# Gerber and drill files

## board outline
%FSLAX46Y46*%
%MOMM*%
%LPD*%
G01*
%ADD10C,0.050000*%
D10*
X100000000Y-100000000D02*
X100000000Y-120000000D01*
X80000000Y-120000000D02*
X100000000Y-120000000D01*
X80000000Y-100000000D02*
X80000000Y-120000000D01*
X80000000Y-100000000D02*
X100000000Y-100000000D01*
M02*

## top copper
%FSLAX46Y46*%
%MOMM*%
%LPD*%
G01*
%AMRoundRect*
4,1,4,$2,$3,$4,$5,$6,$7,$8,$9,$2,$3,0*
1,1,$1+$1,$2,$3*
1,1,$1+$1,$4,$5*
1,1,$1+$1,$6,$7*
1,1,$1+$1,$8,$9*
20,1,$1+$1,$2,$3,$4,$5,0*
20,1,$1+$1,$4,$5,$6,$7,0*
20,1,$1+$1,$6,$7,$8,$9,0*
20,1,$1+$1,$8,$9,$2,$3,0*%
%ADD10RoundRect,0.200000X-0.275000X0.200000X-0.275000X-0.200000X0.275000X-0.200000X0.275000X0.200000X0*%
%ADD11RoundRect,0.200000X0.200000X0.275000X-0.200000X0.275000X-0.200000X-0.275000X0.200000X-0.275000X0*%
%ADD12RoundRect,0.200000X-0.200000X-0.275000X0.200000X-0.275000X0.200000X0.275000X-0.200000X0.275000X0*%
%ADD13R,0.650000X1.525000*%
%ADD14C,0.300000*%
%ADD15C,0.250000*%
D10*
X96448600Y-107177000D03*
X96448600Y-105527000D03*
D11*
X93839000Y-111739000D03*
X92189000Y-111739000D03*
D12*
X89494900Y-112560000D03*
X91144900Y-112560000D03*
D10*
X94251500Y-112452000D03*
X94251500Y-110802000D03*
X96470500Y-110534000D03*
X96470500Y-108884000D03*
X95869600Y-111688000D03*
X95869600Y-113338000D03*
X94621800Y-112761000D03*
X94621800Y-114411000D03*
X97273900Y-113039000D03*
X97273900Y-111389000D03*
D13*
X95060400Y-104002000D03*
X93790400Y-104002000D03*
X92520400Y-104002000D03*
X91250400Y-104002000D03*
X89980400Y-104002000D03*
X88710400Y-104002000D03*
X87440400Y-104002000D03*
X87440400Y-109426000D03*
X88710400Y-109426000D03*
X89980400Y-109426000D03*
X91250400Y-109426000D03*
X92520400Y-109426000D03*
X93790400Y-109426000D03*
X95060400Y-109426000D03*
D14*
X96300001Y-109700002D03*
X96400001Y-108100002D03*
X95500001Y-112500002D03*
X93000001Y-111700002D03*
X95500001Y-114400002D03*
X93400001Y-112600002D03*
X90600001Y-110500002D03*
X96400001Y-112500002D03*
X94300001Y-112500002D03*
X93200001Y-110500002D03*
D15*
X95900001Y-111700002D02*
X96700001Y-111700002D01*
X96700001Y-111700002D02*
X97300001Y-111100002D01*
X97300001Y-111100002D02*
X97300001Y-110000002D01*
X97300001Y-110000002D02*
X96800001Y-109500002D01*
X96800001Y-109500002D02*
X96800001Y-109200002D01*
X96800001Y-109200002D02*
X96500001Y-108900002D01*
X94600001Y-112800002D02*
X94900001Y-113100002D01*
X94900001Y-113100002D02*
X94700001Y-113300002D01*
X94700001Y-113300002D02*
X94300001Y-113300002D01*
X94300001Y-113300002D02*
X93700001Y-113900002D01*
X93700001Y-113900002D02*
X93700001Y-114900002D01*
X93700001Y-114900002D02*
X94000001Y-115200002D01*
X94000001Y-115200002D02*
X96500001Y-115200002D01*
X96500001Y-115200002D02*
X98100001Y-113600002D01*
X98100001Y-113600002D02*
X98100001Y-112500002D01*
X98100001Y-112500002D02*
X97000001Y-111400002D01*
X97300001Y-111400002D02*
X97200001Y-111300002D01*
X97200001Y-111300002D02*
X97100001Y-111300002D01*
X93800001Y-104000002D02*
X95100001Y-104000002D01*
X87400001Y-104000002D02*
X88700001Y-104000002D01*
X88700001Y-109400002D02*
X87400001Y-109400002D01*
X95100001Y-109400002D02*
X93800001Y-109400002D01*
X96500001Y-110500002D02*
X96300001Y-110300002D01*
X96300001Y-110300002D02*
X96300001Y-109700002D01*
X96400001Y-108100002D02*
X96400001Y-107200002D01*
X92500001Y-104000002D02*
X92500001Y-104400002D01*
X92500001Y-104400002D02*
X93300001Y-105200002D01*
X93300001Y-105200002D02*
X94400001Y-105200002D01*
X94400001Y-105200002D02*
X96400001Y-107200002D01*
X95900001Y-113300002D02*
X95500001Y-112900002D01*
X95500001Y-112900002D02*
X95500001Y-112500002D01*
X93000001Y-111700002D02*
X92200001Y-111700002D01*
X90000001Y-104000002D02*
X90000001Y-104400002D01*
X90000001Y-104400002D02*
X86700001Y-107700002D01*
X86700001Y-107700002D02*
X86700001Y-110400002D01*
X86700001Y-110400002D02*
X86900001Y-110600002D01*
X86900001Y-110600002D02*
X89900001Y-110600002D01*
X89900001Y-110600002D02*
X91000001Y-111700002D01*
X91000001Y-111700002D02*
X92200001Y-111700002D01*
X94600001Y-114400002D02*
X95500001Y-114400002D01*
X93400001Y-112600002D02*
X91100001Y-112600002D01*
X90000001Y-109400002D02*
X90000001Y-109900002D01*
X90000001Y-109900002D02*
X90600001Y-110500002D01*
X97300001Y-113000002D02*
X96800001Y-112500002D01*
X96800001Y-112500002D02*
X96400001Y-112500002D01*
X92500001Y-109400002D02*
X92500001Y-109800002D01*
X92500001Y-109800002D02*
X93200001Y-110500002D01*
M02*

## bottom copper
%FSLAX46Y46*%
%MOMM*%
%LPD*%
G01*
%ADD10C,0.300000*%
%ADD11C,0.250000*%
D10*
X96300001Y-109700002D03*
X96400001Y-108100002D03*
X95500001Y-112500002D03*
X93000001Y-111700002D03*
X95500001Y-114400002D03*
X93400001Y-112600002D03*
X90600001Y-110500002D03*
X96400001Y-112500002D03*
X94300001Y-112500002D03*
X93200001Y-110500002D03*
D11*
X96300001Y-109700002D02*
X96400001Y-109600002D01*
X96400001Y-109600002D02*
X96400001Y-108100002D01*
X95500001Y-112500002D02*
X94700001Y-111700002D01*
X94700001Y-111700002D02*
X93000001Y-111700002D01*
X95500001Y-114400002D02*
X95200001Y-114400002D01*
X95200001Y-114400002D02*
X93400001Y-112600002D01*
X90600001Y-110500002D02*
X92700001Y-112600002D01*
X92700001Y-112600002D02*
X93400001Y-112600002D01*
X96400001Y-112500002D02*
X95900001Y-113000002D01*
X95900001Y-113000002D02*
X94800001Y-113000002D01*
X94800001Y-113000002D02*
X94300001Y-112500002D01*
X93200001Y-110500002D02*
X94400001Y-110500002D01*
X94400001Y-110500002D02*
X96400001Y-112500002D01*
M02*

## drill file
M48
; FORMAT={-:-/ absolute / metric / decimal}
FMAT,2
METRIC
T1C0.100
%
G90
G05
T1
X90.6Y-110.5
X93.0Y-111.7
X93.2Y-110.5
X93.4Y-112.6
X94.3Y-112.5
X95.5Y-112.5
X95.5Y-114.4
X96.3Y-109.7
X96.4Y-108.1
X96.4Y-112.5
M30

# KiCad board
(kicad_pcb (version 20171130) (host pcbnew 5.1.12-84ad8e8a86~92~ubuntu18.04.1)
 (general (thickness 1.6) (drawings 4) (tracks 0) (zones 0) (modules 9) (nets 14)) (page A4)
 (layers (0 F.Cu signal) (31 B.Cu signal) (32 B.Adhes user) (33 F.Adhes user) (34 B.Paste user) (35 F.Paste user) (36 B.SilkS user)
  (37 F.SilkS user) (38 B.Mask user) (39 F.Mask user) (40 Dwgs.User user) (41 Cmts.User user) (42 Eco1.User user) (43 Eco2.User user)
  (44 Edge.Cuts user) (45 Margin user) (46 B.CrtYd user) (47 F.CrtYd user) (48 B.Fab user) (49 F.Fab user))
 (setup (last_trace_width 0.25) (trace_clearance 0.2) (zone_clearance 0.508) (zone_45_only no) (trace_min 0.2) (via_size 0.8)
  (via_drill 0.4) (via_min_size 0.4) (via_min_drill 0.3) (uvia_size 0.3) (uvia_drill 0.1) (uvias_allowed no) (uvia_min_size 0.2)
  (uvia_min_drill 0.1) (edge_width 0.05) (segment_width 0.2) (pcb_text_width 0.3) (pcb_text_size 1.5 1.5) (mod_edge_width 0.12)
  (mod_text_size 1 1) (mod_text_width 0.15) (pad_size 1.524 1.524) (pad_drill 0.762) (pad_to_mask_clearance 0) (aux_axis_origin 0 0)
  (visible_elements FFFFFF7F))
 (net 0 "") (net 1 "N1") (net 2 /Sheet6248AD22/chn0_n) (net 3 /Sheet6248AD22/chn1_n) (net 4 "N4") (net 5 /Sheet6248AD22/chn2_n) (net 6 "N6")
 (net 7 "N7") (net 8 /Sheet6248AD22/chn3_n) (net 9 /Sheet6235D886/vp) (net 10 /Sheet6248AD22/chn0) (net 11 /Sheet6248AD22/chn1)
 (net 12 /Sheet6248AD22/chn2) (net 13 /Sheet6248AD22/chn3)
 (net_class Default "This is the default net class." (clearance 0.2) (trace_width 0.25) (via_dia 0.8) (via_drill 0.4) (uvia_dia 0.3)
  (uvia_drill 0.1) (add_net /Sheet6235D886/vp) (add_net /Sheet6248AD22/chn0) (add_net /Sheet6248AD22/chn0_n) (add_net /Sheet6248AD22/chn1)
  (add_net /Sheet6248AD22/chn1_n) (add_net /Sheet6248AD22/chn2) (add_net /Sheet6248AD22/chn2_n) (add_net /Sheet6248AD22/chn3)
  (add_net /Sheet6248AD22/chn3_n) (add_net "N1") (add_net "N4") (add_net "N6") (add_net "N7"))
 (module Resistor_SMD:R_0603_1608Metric (layer F.Cu) (at 96.448600 106.352000 270.000000)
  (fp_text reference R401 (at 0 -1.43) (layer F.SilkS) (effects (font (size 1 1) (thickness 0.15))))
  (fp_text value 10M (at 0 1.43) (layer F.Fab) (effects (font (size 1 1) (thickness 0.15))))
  (pad 2 smd roundrect (at 0.825 0 270.000000) (size 0.8 0.95) (layers F.Cu F.Mask F.Paste) (roundrect_rratio 0.25) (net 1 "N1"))
  (pad 1 smd roundrect (at -0.825 0 270.000000) (size 0.8 0.95) (layers F.Cu F.Mask F.Paste) (roundrect_rratio 0.25)
   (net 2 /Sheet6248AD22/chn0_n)))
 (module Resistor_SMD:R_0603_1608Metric (layer F.Cu) (at 93.014000 111.739000 180.000000)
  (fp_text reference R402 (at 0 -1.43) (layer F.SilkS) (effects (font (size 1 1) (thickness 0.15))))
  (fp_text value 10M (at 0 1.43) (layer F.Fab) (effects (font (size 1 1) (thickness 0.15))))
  (pad 1 smd roundrect (at -0.825 0 180.000000) (size 0.8 0.95) (layers F.Cu F.Mask F.Paste) (roundrect_rratio 0.25)
   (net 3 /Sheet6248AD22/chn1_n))
  (pad 2 smd roundrect (at 0.825 0 180.000000) (size 0.8 0.95) (layers F.Cu F.Mask F.Paste) (roundrect_rratio 0.25) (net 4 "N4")))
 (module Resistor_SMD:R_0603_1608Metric (layer F.Cu) (at 90.319900 112.560000)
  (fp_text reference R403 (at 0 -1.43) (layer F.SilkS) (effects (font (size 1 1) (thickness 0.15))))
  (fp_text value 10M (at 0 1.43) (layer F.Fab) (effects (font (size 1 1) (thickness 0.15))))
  (pad 1 smd roundrect (at -0.825 0) (size 0.8 0.95) (layers F.Cu F.Mask F.Paste) (roundrect_rratio 0.25) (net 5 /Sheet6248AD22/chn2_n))
  (pad 2 smd roundrect (at 0.825 0) (size 0.8 0.95) (layers F.Cu F.Mask F.Paste) (roundrect_rratio 0.25) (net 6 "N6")))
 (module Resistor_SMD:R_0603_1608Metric (layer F.Cu) (at 94.251500 111.627000 270.000000)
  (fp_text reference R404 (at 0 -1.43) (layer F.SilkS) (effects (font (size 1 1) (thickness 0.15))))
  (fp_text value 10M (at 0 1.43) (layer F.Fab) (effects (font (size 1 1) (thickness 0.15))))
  (pad 2 smd roundrect (at 0.825 0 270.000000) (size 0.8 0.95) (layers F.Cu F.Mask F.Paste) (roundrect_rratio 0.25) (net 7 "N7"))
  (pad 1 smd roundrect (at -0.825 0 270.000000) (size 0.8 0.95) (layers F.Cu F.Mask F.Paste) (roundrect_rratio 0.25)
   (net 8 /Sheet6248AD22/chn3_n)))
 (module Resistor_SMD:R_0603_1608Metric (layer F.Cu) (at 96.470500 109.709000 270.000000)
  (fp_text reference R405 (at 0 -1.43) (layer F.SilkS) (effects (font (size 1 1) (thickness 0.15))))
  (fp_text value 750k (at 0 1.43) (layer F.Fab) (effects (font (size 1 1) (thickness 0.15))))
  (pad 2 smd roundrect (at 0.825 0 270.000000) (size 0.8 0.95) (layers F.Cu F.Mask F.Paste) (roundrect_rratio 0.25) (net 1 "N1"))
  (pad 1 smd roundrect (at -0.825 0 270.000000) (size 0.8 0.95) (layers F.Cu F.Mask F.Paste) (roundrect_rratio 0.25)
   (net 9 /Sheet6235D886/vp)))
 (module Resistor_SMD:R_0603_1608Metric (layer F.Cu) (at 95.869600 112.513000 270.000000)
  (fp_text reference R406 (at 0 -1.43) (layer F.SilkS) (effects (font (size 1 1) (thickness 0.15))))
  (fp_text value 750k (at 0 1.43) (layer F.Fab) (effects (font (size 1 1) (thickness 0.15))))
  (pad 1 smd roundrect (at -0.825 0 270.000000) (size 0.8 0.95) (layers F.Cu F.Mask F.Paste) (roundrect_rratio 0.25)
   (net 9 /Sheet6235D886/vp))
  (pad 2 smd roundrect (at 0.825 0 270.000000) (size 0.8 0.95) (layers F.Cu F.Mask F.Paste) (roundrect_rratio 0.25) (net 4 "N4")))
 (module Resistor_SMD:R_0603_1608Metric (layer F.Cu) (at 94.621800 113.586000 270.000000)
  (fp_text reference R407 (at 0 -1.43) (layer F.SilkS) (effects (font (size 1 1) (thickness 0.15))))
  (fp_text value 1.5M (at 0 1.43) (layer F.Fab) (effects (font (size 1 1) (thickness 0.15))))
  (pad 1 smd roundrect (at -0.825 0 270.000000) (size 0.8 0.95) (layers F.Cu F.Mask F.Paste) (roundrect_rratio 0.25)
   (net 9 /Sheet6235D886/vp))
  (pad 2 smd roundrect (at 0.825 0 270.000000) (size 0.8 0.95) (layers F.Cu F.Mask F.Paste) (roundrect_rratio 0.25) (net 6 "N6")))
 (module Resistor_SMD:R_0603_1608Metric (layer F.Cu) (at 97.273900 112.214000 270.000000)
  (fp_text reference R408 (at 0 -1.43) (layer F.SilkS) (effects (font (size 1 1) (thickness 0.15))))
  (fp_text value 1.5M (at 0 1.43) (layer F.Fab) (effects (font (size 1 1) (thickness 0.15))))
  (pad 2 smd roundrect (at 0.825 0 270.000000) (size 0.8 0.95) (layers F.Cu F.Mask F.Paste) (roundrect_rratio 0.25) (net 7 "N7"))
  (pad 1 smd roundrect (at -0.825 0 270.000000) (size 0.8 0.95) (layers F.Cu F.Mask F.Paste) (roundrect_rratio 0.25)
   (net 9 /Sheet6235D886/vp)))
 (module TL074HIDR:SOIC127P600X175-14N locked (layer F.Cu) (at 91.250400 106.714000 270.000000)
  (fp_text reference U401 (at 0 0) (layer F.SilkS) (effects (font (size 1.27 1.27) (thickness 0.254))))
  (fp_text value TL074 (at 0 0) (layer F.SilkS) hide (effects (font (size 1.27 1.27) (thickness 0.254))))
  (pad 1 smd rect (at -2.712 -3.81) (size 0.65 1.525) (layers F.Cu F.Mask F.Paste) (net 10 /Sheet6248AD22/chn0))
  (pad 2 smd rect (at -2.712 -2.54) (size 0.65 1.525) (layers F.Cu F.Mask F.Paste) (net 10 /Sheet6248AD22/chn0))
  (pad 3 smd rect (at -2.712 -1.27) (size 0.65 1.525) (layers F.Cu F.Mask F.Paste) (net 1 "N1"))
  (pad 4 smd rect (at -2.712 0) (size 0.65 1.525) (layers F.Cu F.Mask F.Paste))
  (pad 5 smd rect (at -2.712 1.27) (size 0.65 1.525) (layers F.Cu F.Mask F.Paste) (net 4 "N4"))
  (pad 6 smd rect (at -2.712 2.54) (size 0.65 1.525) (layers F.Cu F.Mask F.Paste) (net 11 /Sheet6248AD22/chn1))
  (pad 7 smd rect (at -2.712 3.81) (size 0.65 1.525) (layers F.Cu F.Mask F.Paste) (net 11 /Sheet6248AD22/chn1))
  (pad 8 smd rect (at 2.712 3.81) (size 0.65 1.525) (layers F.Cu F.Mask F.Paste) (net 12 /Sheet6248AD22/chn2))
  (pad 9 smd rect (at 2.712 2.54) (size 0.65 1.525) (layers F.Cu F.Mask F.Paste) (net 12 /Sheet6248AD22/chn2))
  (pad 10 smd rect (at 2.712 1.27) (size 0.65 1.525) (layers F.Cu F.Mask F.Paste) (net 6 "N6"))
  (pad 11 smd rect (at 2.712 0) (size 0.65 1.525) (layers F.Cu F.Mask F.Paste))
  (pad 12 smd rect (at 2.712 -1.27) (size 0.65 1.525) (layers F.Cu F.Mask F.Paste) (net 7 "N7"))
  (pad 13 smd rect (at 2.712 -2.54) (size 0.65 1.525) (layers F.Cu F.Mask F.Paste) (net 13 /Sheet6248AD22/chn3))
  (pad 14 smd rect (at 2.712 -3.81) (size 0.65 1.525) (layers F.Cu F.Mask F.Paste) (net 13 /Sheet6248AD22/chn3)))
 (gr_line (start 100 100) (end 100 120) (layer Edge.Cuts) (width 0.05))
 (gr_line (start 80 120) (end 100 120) (layer Edge.Cuts) (width 0.05))
 (gr_line (start 80 100) (end 80 120) (layer Edge.Cuts) (width 0.05))
 (gr_line (start 80 100) (end 100 100) (layer Edge.Cuts) (width 0.05))
 (segment (start 95.900001 111.700002) (end 96.700001 111.700002) (width 0.250000) (layer F.Cu) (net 9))
 (segment (start 96.700001 111.700002) (end 97.300001 111.100002) (width 0.250000) (layer F.Cu) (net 9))
 (segment (start 97.300001 111.100002) (end 97.300001 110.000002) (width 0.250000) (layer F.Cu) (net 9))
 (segment (start 97.300001 110.000002) (end 96.800001 109.500002) (width 0.250000) (layer F.Cu) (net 9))
 (segment (start 96.800001 109.500002) (end 96.800001 109.200002) (width 0.250000) (layer F.Cu) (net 9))
 (segment (start 96.800001 109.200002) (end 96.500001 108.900002) (width 0.250000) (layer F.Cu) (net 9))
 (segment (start 94.600001 112.800002) (end 94.900001 113.100002) (width 0.250000) (layer F.Cu) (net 9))
 (segment (start 94.900001 113.100002) (end 94.700001 113.300002) (width 0.250000) (layer F.Cu) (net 9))
 (segment (start 94.700001 113.300002) (end 94.300001 113.300002) (width 0.250000) (layer F.Cu) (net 9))
 (segment (start 94.300001 113.300002) (end 93.700001 113.900002) (width 0.250000) (layer F.Cu) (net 9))
 (segment (start 93.700001 113.900002) (end 93.700001 114.900002) (width 0.250000) (layer F.Cu) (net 9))
 (segment (start 93.700001 114.900002) (end 94.000001 115.200002) (width 0.250000) (layer F.Cu) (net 9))
 (segment (start 94.000001 115.200002) (end 96.500001 115.200002) (width 0.250000) (layer F.Cu) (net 9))
 (segment (start 96.500001 115.200002) (end 98.100001 113.600002) (width 0.250000) (layer F.Cu) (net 9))
 (segment (start 98.100001 113.600002) (end 98.100001 112.500002) (width 0.250000) (layer F.Cu) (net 9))
 (segment (start 98.100001 112.500002) (end 97.000001 111.400002) (width 0.250000) (layer F.Cu) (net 9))
 (segment (start 97.300001 111.400002) (end 97.200001 111.300002) (width 0.250000) (layer F.Cu) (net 9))
 (segment (start 97.200001 111.300002) (end 97.100001 111.300002) (width 0.250000) (layer F.Cu) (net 9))
 (segment (start 93.800001 104.000002) (end 95.100001 104.000002) (width 0.250000) (layer F.Cu) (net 10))
 (segment (start 87.400001 104.000002) (end 88.700001 104.000002) (width 0.250000) (layer F.Cu) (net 11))
 (segment (start 88.700001 109.400002) (end 87.400001 109.400002) (width 0.250000) (layer F.Cu) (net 12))
 (segment (start 95.100001 109.400002) (end 93.800001 109.400002) (width 0.250000) (layer F.Cu) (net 13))
 (segment (start 96.500001 110.500002) (end 96.300001 110.300002) (width 0.250000) (layer F.Cu) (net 1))
 (segment (start 96.300001 110.300002) (end 96.300001 109.700002) (width 0.250000) (layer F.Cu) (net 1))
 (segment (start 96.300001 109.700002) (end 96.400001 109.600002) (width 0.250000) (layer B.Cu) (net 1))
 (segment (start 96.400001 109.600002) (end 96.400001 108.100002) (width 0.250000) (layer B.Cu) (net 1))
 (segment (start 96.400001 108.100002) (end 96.400001 107.200002) (width 0.250000) (layer F.Cu) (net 1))
 (segment (start 92.500001 104.000002) (end 92.500001 104.400002) (width 0.250000) (layer F.Cu) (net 1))
 (segment (start 92.500001 104.400002) (end 93.300001 105.200002) (width 0.250000) (layer F.Cu) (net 1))
 (segment (start 93.300001 105.200002) (end 94.400001 105.200002) (width 0.250000) (layer F.Cu) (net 1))
 (segment (start 94.400001 105.200002) (end 96.400001 107.200002) (width 0.250000) (layer F.Cu) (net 1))
 (via micro (at 96.300001 109.700002) (size 0.300000) (drill 0.100000) (layers F.Cu B.Cu) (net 1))
 (via micro (at 96.400001 108.100002) (size 0.300000) (drill 0.100000) (layers F.Cu B.Cu) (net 1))
 (segment (start 95.900001 113.300002) (end 95.500001 112.900002) (width 0.250000) (layer F.Cu) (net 4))
 (segment (start 95.500001 112.900002) (end 95.500001 112.500002) (width 0.250000) (layer F.Cu) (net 4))
 (segment (start 95.500001 112.500002) (end 94.700001 111.700002) (width 0.250000) (layer B.Cu) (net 4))
 (segment (start 94.700001 111.700002) (end 93.000001 111.700002) (width 0.250000) (layer B.Cu) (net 4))
 (segment (start 93.000001 111.700002) (end 92.200001 111.700002) (width 0.250000) (layer F.Cu) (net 4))
 (segment (start 90.000001 104.000002) (end 90.000001 104.400002) (width 0.250000) (layer F.Cu) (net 4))
 (segment (start 90.000001 104.400002) (end 86.700001 107.700002) (width 0.250000) (layer F.Cu) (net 4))
 (segment (start 86.700001 107.700002) (end 86.700001 110.400002) (width 0.250000) (layer F.Cu) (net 4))
 (segment (start 86.700001 110.400002) (end 86.900001 110.600002) (width 0.250000) (layer F.Cu) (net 4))
 (segment (start 86.900001 110.600002) (end 89.900001 110.600002) (width 0.250000) (layer F.Cu) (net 4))
 (segment (start 89.900001 110.600002) (end 91.000001 111.700002) (width 0.250000) (layer F.Cu) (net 4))
 (segment (start 91.000001 111.700002) (end 92.200001 111.700002) (width 0.250000) (layer F.Cu) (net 4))
 (via micro (at 95.500001 112.500002) (size 0.300000) (drill 0.100000) (layers F.Cu B.Cu) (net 4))
 (via micro (at 93.000001 111.700002) (size 0.300000) (drill 0.100000) (layers F.Cu B.Cu) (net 4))
 (segment (start 94.600001 114.400002) (end 95.500001 114.400002) (width 0.250000) (layer F.Cu) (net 6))
 (segment (start 95.500001 114.400002) (end 95.200001 114.400002) (width 0.250000) (layer B.Cu) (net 6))
 (segment (start 95.200001 114.400002) (end 93.400001 112.600002) (width 0.250000) (layer B.Cu) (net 6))
 (segment (start 93.400001 112.600002) (end 91.100001 112.600002) (width 0.250000) (layer F.Cu) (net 6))
 (segment (start 90.000001 109.400002) (end 90.000001 109.900002) (width 0.250000) (layer F.Cu) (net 6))
 (segment (start 90.000001 109.900002) (end 90.600001 110.500002) (width 0.250000) (layer F.Cu) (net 6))
 (segment (start 90.600001 110.500002) (end 92.700001 112.600002) (width 0.250000) (layer B.Cu) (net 6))
 (segment (start 92.700001 112.600002) (end 93.400001 112.600002) (width 0.250000) (layer B.Cu) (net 6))
 (via micro (at 95.500001 114.400002) (size 0.300000) (drill 0.100000) (layers F.Cu B.Cu) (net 6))
 (via micro (at 93.400001 112.600002) (size 0.300000) (drill 0.100000) (layers F.Cu B.Cu) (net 6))
 (via micro (at 90.600001 110.500002) (size 0.300000) (drill 0.100000) (layers F.Cu B.Cu) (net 6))
 (segment (start 97.300001 113.000002) (end 96.800001 112.500002) (width 0.250000) (layer F.Cu) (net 7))
 (segment (start 96.800001 112.500002) (end 96.400001 112.500002) (width 0.250000) (layer F.Cu) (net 7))
 (segment (start 96.400001 112.500002) (end 95.900001 113.000002) (width 0.250000) (layer B.Cu) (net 7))
 (segment (start 95.900001 113.000002) (end 94.800001 113.000002) (width 0.250000) (layer B.Cu) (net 7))
 (segment (start 94.800001 113.000002) (end 94.300001 112.500002) (width 0.250000) (layer B.Cu) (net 7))
 (segment (start 92.500001 109.400002) (end 92.500001 109.800002) (width 0.250000) (layer F.Cu) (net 7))
 (segment (start 92.500001 109.800002) (end 93.200001 110.500002) (width 0.250000) (layer F.Cu) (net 7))
 (segment (start 93.200001 110.500002) (end 94.400001 110.500002) (width 0.250000) (layer B.Cu) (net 7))
 (segment (start 94.400001 110.500002) (end 96.400001 112.500002) (width 0.250000) (layer B.Cu) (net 7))
 (via micro (at 96.400001 112.500002) (size 0.300000) (drill 0.100000) (layers F.Cu B.Cu) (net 7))
 (via micro (at 94.300001 112.500002) (size 0.300000) (drill 0.100000) (layers F.Cu B.Cu) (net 7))
 (via micro (at 93.200001 110.500002) (size 0.300000) (drill 0.100000) (layers F.Cu B.Cu) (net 7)))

